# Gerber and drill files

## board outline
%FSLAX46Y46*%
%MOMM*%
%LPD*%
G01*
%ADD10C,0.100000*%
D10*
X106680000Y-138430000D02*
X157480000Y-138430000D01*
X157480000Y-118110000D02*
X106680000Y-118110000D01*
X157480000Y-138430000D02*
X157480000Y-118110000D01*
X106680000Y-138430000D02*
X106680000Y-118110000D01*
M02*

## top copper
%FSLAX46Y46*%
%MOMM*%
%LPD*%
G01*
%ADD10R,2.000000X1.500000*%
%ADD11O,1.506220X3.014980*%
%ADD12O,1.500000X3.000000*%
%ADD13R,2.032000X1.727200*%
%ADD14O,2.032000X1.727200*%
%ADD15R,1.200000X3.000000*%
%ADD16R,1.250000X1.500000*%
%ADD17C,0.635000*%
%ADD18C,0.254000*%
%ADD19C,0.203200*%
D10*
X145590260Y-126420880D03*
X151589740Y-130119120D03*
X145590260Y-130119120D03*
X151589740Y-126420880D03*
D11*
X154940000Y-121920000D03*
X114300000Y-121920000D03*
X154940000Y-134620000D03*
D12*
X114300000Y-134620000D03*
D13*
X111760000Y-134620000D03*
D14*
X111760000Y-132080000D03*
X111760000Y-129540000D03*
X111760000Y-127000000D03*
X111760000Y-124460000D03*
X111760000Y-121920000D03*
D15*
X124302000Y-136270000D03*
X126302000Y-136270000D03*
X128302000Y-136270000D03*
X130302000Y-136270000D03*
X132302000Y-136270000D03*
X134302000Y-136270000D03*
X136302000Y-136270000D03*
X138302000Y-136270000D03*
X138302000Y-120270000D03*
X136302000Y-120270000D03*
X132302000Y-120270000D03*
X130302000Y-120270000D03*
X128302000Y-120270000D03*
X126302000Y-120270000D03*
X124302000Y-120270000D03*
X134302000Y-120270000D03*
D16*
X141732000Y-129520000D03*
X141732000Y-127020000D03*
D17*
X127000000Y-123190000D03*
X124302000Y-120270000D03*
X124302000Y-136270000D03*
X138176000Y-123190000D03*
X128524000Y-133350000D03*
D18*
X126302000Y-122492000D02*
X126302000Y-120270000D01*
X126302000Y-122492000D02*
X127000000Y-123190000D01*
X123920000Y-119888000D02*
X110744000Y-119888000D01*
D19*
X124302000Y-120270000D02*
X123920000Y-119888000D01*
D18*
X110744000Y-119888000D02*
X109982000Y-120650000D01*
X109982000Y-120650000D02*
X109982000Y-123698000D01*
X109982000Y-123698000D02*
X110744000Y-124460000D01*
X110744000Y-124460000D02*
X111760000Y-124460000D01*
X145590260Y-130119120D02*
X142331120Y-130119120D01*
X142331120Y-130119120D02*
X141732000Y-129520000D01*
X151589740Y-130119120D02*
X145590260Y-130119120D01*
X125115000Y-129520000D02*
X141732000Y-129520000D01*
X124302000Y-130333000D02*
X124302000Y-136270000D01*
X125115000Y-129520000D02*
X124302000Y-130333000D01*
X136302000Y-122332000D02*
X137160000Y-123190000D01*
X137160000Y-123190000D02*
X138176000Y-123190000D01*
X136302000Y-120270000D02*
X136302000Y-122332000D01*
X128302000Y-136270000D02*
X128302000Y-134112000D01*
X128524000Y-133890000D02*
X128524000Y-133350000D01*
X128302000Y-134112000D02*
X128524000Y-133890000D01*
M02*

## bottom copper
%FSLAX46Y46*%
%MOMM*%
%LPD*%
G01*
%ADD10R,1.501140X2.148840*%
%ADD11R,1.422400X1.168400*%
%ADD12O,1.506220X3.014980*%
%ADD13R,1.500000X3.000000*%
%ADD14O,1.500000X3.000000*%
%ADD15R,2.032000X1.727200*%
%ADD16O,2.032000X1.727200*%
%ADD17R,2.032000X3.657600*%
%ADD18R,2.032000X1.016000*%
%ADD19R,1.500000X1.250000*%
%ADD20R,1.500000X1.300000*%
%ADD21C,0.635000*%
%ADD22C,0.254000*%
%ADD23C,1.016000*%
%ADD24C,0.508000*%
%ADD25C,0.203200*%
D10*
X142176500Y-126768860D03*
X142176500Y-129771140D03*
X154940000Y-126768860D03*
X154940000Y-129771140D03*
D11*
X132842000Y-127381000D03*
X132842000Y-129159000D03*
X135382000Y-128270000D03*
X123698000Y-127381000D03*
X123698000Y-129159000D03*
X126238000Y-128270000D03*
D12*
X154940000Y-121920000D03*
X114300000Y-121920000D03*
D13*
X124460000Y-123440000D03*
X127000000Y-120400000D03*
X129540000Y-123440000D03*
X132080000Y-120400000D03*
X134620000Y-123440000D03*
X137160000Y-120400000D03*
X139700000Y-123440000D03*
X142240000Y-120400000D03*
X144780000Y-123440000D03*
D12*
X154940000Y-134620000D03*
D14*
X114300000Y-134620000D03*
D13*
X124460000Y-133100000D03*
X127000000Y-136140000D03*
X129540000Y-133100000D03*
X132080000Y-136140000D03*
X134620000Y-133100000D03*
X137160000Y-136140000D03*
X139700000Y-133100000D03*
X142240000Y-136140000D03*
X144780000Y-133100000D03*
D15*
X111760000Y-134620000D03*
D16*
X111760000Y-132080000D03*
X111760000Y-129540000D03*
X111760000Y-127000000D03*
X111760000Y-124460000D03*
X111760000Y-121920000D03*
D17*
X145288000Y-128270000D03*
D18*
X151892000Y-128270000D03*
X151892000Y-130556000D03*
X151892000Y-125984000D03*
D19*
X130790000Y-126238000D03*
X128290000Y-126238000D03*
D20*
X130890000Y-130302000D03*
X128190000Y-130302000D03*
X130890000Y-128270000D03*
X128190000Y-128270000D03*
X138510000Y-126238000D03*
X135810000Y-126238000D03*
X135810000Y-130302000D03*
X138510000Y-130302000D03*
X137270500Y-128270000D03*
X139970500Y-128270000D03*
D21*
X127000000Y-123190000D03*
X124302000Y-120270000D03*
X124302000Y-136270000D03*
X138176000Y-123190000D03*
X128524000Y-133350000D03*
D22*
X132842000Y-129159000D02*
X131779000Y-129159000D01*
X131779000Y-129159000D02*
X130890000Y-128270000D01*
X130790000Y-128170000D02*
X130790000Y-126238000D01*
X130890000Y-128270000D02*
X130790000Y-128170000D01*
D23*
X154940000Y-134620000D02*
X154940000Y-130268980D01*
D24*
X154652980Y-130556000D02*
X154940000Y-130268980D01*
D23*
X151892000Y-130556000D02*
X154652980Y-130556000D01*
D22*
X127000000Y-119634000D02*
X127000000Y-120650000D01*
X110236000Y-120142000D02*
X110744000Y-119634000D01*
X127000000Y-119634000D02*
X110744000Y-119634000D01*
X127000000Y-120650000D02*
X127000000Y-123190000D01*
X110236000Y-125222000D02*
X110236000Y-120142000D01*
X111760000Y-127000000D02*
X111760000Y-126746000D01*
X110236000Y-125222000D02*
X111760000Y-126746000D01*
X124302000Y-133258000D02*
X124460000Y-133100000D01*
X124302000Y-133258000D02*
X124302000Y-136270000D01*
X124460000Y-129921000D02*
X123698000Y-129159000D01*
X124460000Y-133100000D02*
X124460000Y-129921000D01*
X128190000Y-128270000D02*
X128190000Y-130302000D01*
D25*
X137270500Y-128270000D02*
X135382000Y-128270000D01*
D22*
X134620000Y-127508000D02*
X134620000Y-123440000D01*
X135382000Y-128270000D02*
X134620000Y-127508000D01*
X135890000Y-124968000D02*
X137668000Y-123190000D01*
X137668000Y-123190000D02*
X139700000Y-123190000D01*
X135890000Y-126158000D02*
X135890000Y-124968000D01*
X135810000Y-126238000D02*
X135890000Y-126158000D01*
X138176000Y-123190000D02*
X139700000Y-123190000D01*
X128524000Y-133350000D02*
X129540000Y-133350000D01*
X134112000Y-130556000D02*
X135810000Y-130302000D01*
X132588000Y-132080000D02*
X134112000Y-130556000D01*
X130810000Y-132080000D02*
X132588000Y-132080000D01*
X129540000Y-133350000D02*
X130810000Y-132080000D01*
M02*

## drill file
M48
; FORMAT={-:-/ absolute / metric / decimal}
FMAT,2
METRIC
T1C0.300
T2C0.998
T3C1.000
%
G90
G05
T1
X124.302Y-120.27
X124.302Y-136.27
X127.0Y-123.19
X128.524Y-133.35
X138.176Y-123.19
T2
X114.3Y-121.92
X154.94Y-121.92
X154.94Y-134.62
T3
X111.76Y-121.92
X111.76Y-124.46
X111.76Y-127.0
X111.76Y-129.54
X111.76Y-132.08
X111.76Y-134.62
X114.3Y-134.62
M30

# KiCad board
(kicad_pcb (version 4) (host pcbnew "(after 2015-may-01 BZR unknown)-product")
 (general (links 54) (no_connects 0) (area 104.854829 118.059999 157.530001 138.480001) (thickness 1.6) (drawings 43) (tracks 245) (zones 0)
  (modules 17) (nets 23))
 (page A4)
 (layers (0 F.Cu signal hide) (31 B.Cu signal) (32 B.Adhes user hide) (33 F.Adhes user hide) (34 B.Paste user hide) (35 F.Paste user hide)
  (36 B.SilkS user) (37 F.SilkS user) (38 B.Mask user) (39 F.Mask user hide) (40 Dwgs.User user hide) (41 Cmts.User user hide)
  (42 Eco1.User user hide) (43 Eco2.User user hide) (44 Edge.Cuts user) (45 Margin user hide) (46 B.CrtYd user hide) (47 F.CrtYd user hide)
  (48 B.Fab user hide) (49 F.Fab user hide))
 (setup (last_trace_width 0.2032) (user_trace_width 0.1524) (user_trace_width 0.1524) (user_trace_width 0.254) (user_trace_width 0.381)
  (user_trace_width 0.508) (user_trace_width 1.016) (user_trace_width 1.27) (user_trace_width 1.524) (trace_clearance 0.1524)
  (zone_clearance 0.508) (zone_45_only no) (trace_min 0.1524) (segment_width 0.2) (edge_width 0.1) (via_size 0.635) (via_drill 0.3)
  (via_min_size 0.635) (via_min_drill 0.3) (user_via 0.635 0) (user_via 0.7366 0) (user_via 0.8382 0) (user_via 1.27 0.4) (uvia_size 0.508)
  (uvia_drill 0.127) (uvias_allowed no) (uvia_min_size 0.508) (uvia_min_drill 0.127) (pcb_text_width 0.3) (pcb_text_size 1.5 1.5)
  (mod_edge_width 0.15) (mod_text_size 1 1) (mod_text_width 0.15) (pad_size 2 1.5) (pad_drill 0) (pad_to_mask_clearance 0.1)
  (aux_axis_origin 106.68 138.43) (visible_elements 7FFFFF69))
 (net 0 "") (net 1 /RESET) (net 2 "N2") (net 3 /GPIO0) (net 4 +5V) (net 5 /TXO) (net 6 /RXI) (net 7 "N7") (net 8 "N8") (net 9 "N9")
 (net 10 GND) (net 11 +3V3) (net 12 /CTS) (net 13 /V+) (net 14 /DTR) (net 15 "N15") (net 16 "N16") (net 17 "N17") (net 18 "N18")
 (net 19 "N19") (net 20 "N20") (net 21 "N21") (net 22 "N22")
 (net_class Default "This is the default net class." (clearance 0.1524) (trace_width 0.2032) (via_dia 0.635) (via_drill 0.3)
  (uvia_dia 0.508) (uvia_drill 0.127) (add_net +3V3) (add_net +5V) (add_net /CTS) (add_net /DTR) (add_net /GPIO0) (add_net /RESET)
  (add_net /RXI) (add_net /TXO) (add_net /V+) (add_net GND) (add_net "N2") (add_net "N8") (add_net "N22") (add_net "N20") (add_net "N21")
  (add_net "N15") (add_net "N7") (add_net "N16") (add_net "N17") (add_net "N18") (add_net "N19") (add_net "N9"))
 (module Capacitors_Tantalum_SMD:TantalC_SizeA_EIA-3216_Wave (layer B.Cu) (at 142.1765 128.27 90)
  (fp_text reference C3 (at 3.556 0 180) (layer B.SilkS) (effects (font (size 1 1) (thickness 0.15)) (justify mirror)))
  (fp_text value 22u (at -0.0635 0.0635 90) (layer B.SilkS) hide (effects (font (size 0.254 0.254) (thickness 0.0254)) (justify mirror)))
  (pad 2 smd rect (at 1.50114 0 90) (size 2.14884 1.50114) (layers B.Cu B.Paste B.Mask))
  (pad 1 smd rect (at -1.50114 0 90) (size 2.14884 1.50114) (layers B.Cu B.Paste B.Mask)))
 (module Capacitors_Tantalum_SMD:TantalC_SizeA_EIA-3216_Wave (layer B.Cu) (at 154.94 128.27 90)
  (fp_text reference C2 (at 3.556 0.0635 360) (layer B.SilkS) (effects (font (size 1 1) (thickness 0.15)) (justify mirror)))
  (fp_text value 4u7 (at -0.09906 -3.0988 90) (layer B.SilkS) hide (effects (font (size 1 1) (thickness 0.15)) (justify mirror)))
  (pad 2 smd rect (at 1.50114 0 90) (size 2.14884 1.50114) (layers B.Cu B.Paste B.Mask))
  (pad 1 smd rect (at -1.50114 0 90) (size 2.14884 1.50114) (layers B.Cu B.Paste B.Mask)))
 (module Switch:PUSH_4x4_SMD (layer F.Cu) (at 148.59 128.27) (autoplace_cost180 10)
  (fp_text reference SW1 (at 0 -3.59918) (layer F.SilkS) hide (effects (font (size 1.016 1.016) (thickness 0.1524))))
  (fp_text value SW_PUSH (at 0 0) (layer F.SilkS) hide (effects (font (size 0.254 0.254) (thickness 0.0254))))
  (pad 1 smd rect (at -2.99974 -1.84912) (size 2 1.5) (layers F.Cu F.Paste F.Mask))
  (pad 2 smd rect (at 2.99974 1.84912) (size 2 1.5) (layers F.Cu F.Paste F.Mask) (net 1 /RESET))
  (pad 2 smd rect (at -2.99974 1.84912) (size 2 1.5) (layers F.Cu F.Paste F.Mask) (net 1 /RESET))
  (pad 1 smd rect (at 2.99974 -1.84912) (size 2 1.5) (layers F.Cu F.Paste F.Mask)))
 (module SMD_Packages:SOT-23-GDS (layer B.Cu) (at 134.112 128.27 270)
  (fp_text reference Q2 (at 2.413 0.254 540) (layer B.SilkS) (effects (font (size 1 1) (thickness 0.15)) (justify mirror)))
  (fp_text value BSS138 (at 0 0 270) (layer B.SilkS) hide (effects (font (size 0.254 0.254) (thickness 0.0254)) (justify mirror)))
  (pad S smd rect (at -0.889 1.27 270) (size 1.1684 1.4224) (layers B.Cu B.Paste B.Mask))
  (pad G smd rect (at 0.889 1.27 270) (size 1.1684 1.4224) (layers B.Cu B.Paste B.Mask) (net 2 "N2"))
  (pad D smd rect (at 0 -1.27 270) (size 1.1684 1.4224) (layers B.Cu B.Paste B.Mask) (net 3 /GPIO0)))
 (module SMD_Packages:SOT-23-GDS (layer B.Cu) (at 124.968 128.27 270)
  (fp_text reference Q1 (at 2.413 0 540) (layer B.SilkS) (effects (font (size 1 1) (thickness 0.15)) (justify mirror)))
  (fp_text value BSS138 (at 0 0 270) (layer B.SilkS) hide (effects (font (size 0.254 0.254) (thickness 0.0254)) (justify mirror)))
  (pad S smd rect (at -0.889 1.27 270) (size 1.1684 1.4224) (layers B.Cu B.Paste B.Mask))
  (pad G smd rect (at 0.889 1.27 270) (size 1.1684 1.4224) (layers B.Cu B.Paste B.Mask) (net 1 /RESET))
  (pad D smd rect (at 0 -1.27 270) (size 1.1684 1.4224) (layers B.Cu B.Paste B.Mask)))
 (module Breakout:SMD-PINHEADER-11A (layer B.Cu) (at 114.3 121.92)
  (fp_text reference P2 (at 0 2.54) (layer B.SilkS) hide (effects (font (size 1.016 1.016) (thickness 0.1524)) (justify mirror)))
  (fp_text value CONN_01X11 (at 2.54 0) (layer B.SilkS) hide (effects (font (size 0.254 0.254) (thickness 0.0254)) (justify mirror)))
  (pad 11 thru_hole oval (at 40.64 0) (size 1.50622 3.01498) (drill 0.99822) (layers *.Cu *.Mask))
  (pad 1 thru_hole oval (at 0 0) (size 1.50622 3.01498) (drill 0.99822) (layers *.Cu *.Mask))
  (pad 2 smd rect (at 10.16 1.52) (size 1.5 3) (layers B.Cu B.Paste B.Mask))
  (pad 3 smd rect (at 12.7 -1.52) (size 1.5 3) (layers B.Cu B.Paste B.Mask))
  (pad 4 smd rect (at 15.24 1.52) (size 1.5 3) (layers B.Cu B.Paste B.Mask))
  (pad 5 smd rect (at 17.78 -1.52) (size 1.5 3) (layers B.Cu B.Paste B.Mask))
  (pad 6 smd rect (at 20.32 1.52) (size 1.5 3) (layers B.Cu B.Paste B.Mask) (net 3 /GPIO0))
  (pad 7 smd rect (at 22.86 -1.52) (size 1.5 3) (layers B.Cu B.Paste B.Mask))
  (pad 8 smd rect (at 25.4 1.52) (size 1.5 3) (layers B.Cu B.Paste B.Mask))
  (pad 9 smd rect (at 27.94 -1.52) (size 1.5 3) (layers B.Cu B.Paste B.Mask))
  (pad 10 smd rect (at 30.48 1.52) (size 1.5 3) (layers B.Cu B.Paste B.Mask)))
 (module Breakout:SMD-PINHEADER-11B (layer B.Cu) (at 114.3 134.62)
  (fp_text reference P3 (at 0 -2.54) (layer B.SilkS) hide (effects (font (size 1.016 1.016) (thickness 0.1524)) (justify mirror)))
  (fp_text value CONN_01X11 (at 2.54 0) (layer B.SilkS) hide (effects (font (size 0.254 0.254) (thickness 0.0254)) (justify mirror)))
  (pad 11 thru_hole oval (at 40.64 0) (size 1.50622 3.01498) (drill 0.99822) (layers *.Cu *.Mask) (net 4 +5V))
  (pad 1 thru_hole oval (at 0 0) (size 1.5 3) (drill 1) (layers *.Cu *.Mask))
  (pad 2 smd rect (at 10.16 -1.52) (size 1.5 3) (layers B.Cu B.Paste B.Mask) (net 1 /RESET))
  (pad 3 smd rect (at 12.7 1.52) (size 1.5 3) (layers B.Cu B.Paste B.Mask))
  (pad 4 smd rect (at 15.24 -1.52) (size 1.5 3) (layers B.Cu B.Paste B.Mask))
  (pad 5 smd rect (at 17.78 1.52) (size 1.5 3) (layers B.Cu B.Paste B.Mask))
  (pad 6 smd rect (at 20.32 -1.52) (size 1.5 3) (layers B.Cu B.Paste B.Mask))
  (pad 7 smd rect (at 22.86 1.52) (size 1.5 3) (layers B.Cu B.Paste B.Mask))
  (pad 8 smd rect (at 25.4 -1.52) (size 1.5 3) (layers B.Cu B.Paste B.Mask))
  (pad 9 smd rect (at 27.94 1.52) (size 1.5 3) (layers B.Cu B.Paste B.Mask))
  (pad 10 smd rect (at 30.48 -1.52) (size 1.5 3) (layers B.Cu B.Paste B.Mask)))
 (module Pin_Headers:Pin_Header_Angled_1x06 (layer F.Cu) (at 111.76 128.27 90)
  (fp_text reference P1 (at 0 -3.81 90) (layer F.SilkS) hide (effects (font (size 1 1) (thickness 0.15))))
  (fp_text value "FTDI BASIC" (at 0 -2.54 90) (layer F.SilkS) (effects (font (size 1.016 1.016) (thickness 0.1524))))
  (pad 1 thru_hole rect (at -6.35 0 90) (size 1.7272 2.032) (drill 1) (layers *.Cu *.Mask F.SilkS))
  (pad 2 thru_hole oval (at -3.81 0 90) (size 1.7272 2.032) (drill 1) (layers *.Cu *.Mask F.SilkS))
  (pad 3 thru_hole oval (at -1.27 0 90) (size 1.7272 2.032) (drill 1) (layers *.Cu *.Mask F.SilkS))
  (pad 4 thru_hole oval (at 1.27 0 90) (size 1.7272 2.032) (drill 1) (layers *.Cu *.Mask F.SilkS) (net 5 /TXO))
  (pad 5 thru_hole oval (at 3.81 0 90) (size 1.7272 2.032) (drill 1) (layers *.Cu *.Mask F.SilkS) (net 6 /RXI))
  (pad 6 thru_hole oval (at 6.35 0 90) (size 1.7272 2.032) (drill 1) (layers *.Cu *.Mask F.SilkS)))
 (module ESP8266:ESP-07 (layer F.Cu) (at 130.302 128.27)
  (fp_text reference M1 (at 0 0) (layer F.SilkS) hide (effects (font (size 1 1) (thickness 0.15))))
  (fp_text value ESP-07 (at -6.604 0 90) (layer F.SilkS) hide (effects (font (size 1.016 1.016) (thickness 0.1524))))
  (pad 1 smd rect (at -6 8) (size 1.2 3) (layers F.Cu F.Paste F.Mask) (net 1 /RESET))
  (pad 2 smd rect (at -4 8) (size 1.2 3) (layers F.Cu F.Paste F.Mask))
  (pad 3 smd rect (at -2 8) (size 1.2 3) (layers F.Cu F.Paste F.Mask) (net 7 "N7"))
  (pad 4 smd rect (at 0 8) (size 1.2 3) (layers F.Cu F.Paste F.Mask))
  (pad 5 smd rect (at 2 8) (size 1.2 3) (layers F.Cu F.Paste F.Mask))
  (pad 6 smd rect (at 4 8) (size 1.2 3) (layers F.Cu F.Paste F.Mask))
  (pad 7 smd rect (at 6 8) (size 1.2 3) (layers F.Cu F.Paste F.Mask))
  (pad 8 smd rect (at 8 8) (size 1.2 3) (layers F.Cu F.Paste F.Mask))
  (pad 9 smd rect (at 8 -8) (size 1.2 3) (layers F.Cu F.Paste F.Mask))
  (pad 10 smd rect (at 6 -8) (size 1.2 3) (layers F.Cu F.Paste F.Mask) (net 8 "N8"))
  (pad 12 smd rect (at 2 -8) (size 1.2 3) (layers F.Cu F.Paste F.Mask))
  (pad 13 smd rect (at 0 -8) (size 1.2 3) (layers F.Cu F.Paste F.Mask))
  (pad 14 smd rect (at -2 -8) (size 1.2 3) (layers F.Cu F.Paste F.Mask))
  (pad 15 smd rect (at -4 -8) (size 1.2 3) (layers F.Cu F.Paste F.Mask) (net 5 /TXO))
  (pad 16 smd rect (at -6 -8) (size 1.2 3) (layers F.Cu F.Paste F.Mask) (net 6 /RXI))
  (pad 11 smd rect (at 4 -8) (size 1.2 3) (layers F.Cu F.Paste F.Mask)))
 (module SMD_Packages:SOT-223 (layer B.Cu) (at 148.59 128.27 270)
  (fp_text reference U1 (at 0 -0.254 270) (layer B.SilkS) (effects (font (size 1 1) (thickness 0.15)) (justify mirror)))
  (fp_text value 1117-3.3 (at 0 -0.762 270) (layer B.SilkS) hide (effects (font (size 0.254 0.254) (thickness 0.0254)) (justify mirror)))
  (pad 2 smd rect (at 0 3.302 270) (size 3.6576 2.032) (layers B.Cu B.Paste B.Mask))
  (pad 2 smd rect (at 0 -3.302 270) (size 1.016 2.032) (layers B.Cu B.Paste B.Mask))
  (pad 3 smd rect (at 2.286 -3.302 270) (size 1.016 2.032) (layers B.Cu B.Paste B.Mask) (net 4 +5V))
  (pad 1 smd rect (at -2.286 -3.302 270) (size 1.016 2.032) (layers B.Cu B.Paste B.Mask)))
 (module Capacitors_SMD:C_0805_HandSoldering (layer B.Cu) (at 129.54 126.238 180)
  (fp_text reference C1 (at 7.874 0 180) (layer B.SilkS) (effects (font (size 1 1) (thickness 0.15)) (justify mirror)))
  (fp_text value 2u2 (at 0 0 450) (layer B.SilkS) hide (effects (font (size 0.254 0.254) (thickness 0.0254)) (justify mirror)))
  (pad 1 smd rect (at -1.25 0 180) (size 1.5 1.25) (layers B.Cu B.Paste B.Mask) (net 2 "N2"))
  (pad 2 smd rect (at 1.25 0 180) (size 1.5 1.25) (layers B.Cu B.Paste B.Mask)))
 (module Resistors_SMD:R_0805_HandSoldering (layer B.Cu) (at 129.54 130.302 180)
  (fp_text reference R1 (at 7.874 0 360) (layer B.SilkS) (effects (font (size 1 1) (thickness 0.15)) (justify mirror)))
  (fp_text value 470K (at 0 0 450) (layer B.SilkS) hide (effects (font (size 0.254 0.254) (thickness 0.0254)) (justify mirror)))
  (pad 1 smd rect (at -1.35 0 180) (size 1.5 1.3) (layers B.Cu B.Paste B.Mask))
  (pad 2 smd rect (at 1.35 0 180) (size 1.5 1.3) (layers B.Cu B.Paste B.Mask) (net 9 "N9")))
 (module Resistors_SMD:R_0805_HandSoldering (layer B.Cu) (at 129.54 128.27 180)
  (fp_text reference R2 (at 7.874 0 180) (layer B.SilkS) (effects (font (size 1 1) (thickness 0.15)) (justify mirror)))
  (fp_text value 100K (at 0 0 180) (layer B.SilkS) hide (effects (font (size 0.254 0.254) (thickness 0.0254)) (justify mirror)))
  (pad 1 smd rect (at -1.35 0 180) (size 1.5 1.3) (layers B.Cu B.Paste B.Mask) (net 2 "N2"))
  (pad 2 smd rect (at 1.35 0 180) (size 1.5 1.3) (layers B.Cu B.Paste B.Mask) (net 9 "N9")))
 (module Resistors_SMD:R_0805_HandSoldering (layer B.Cu) (at 137.16 126.238 180)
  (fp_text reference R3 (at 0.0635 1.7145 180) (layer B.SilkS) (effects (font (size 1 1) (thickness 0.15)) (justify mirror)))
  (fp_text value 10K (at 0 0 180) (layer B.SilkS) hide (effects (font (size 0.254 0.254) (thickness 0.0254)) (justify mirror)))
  (pad 1 smd rect (at -1.35 0 180) (size 1.5 1.3) (layers B.Cu B.Paste B.Mask))
  (pad 2 smd rect (at 1.35 0 180) (size 1.5 1.3) (layers B.Cu B.Paste B.Mask) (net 8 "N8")))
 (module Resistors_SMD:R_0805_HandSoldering (layer B.Cu) (at 137.16 130.302)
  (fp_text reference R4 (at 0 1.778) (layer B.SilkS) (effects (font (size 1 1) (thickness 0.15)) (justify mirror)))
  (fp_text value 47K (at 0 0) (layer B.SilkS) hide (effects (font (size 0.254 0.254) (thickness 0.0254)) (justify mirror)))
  (pad 1 smd rect (at -1.35 0) (size 1.5 1.3) (layers B.Cu B.Paste B.Mask) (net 7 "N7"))
  (pad 2 smd rect (at 1.35 0) (size 1.5 1.3) (layers B.Cu B.Paste B.Mask)))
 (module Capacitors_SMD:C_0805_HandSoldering (layer F.Cu) (at 141.732 128.27 90)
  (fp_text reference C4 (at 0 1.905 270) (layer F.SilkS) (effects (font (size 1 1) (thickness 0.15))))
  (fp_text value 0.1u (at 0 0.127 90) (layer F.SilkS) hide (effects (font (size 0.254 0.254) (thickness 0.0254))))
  (pad 1 smd rect (at -1.25 0 90) (size 1.5 1.25) (layers F.Cu F.Paste F.Mask) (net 1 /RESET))
  (pad 2 smd rect (at 1.25 0 90) (size 1.5 1.25) (layers F.Cu F.Paste F.Mask)))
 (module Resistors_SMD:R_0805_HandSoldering (layer B.Cu) (at 138.6205 128.27)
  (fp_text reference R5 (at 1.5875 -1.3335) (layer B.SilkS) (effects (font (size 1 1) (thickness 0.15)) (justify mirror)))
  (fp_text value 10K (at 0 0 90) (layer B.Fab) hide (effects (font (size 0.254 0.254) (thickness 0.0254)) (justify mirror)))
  (pad 1 smd rect (at -1.35 0) (size 1.5 1.3) (layers B.Cu B.Paste B.Mask) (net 3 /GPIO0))
  (pad 2 smd rect (at 1.35 0) (size 1.5 1.3) (layers B.Cu B.Paste B.Mask)))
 (gr_line (start 106.68 138.43) (end 157.48 138.43) (angle 90) (layer Edge.Cuts) (width 0.1))
 (gr_line (start 157.48 118.11) (end 106.68 118.11) (angle 90) (layer Edge.Cuts) (width 0.1))
 (gr_line (start 157.48 138.43) (end 157.48 118.11) (angle 90) (layer Edge.Cuts) (width 0.1))
 (gr_line (start 106.68 138.43) (end 106.68 118.11) (angle 90) (layer Edge.Cuts) (width 0.1))
 (segment (start 132.842 129.159) (end 131.779 129.159) (width 0.254) (layer B.Cu) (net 2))
 (segment (start 131.779 129.159) (end 130.89 128.27) (width 0.254) (layer B.Cu) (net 2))
 (segment (start 130.79 128.17) (end 130.79 126.238) (width 0.254) (layer B.Cu) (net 2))
 (segment (start 130.89 128.27) (end 130.79 128.17) (width 0.254) (layer B.Cu) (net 2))
 (segment (start 154.94 134.62) (end 154.94 130.26898) (width 1.016) (layer B.Cu) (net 4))
 (segment (start 154.65298 130.556) (end 154.94 130.26898) (width 0.508) (layer B.Cu) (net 4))
 (segment (start 151.892 130.556) (end 154.65298 130.556) (width 1.016) (layer B.Cu) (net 4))
 (segment (start 127 119.634) (end 127 120.65) (width 0.254) (layer B.Cu) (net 5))
 (segment (start 110.236 120.142) (end 110.744 119.634) (width 0.254) (layer B.Cu) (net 5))
 (segment (start 127 119.634) (end 110.744 119.634) (width 0.254) (layer B.Cu) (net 5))
 (segment (start 126.302 122.492) (end 126.302 120.27) (width 0.254) (layer F.Cu) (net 5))
 (segment (start 126.302 122.492) (end 127 123.19) (width 0.254) (layer F.Cu) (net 5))
 (segment (start 127 120.65) (end 127 123.19) (width 0.254) (layer B.Cu) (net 5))
 (segment (start 110.236 125.222) (end 110.236 120.142) (width 0.254) (layer B.Cu) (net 5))
 (segment (start 111.76 127) (end 111.76 126.746) (width 0.254) (layer B.Cu) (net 5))
 (segment (start 110.236 125.222) (end 111.76 126.746) (width 0.254) (layer B.Cu) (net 5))
 (segment (start 123.92 119.888) (end 110.744 119.888) (width 0.254) (layer F.Cu) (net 6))
 (segment (start 124.302 120.27) (end 123.92 119.888) (width 0.2032) (layer F.Cu) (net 6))
 (segment (start 110.744 119.888) (end 109.982 120.65) (width 0.254) (layer F.Cu) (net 6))
 (segment (start 109.982 120.65) (end 109.982 123.698) (width 0.254) (layer F.Cu) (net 6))
 (segment (start 109.982 123.698) (end 110.744 124.46) (width 0.254) (layer F.Cu) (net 6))
 (segment (start 110.744 124.46) (end 111.76 124.46) (width 0.254) (layer F.Cu) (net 6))
 (segment (start 145.59026 130.11912) (end 142.33112 130.11912) (width 0.254) (layer F.Cu) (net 1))
 (segment (start 142.33112 130.11912) (end 141.732 129.52) (width 0.254) (layer F.Cu) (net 1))
 (segment (start 151.58974 130.11912) (end 145.59026 130.11912) (width 0.254) (layer F.Cu) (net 1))
 (segment (start 124.302 133.258) (end 124.46 133.1) (width 0.254) (layer B.Cu) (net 1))
 (segment (start 125.115 129.52) (end 141.732 129.52) (width 0.254) (layer F.Cu) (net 1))
 (segment (start 124.302 130.333) (end 124.302 136.27) (width 0.254) (layer F.Cu) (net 1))
 (segment (start 125.115 129.52) (end 124.302 130.333) (width 0.254) (layer F.Cu) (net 1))
 (segment (start 124.302 133.258) (end 124.302 136.27) (width 0.254) (layer B.Cu) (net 1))
 (segment (start 124.46 129.921) (end 123.698 129.159) (width 0.254) (layer B.Cu) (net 1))
 (segment (start 124.46 133.1) (end 124.46 129.921) (width 0.254) (layer B.Cu) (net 1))
 (segment (start 128.19 128.27) (end 128.19 130.302) (width 0.254) (layer B.Cu) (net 9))
 (segment (start 137.2705 128.27) (end 135.382 128.27) (width 0.2032) (layer B.Cu) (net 3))
 (segment (start 134.62 127.508) (end 134.62 123.44) (width 0.254) (layer B.Cu) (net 3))
 (segment (start 135.382 128.27) (end 134.62 127.508) (width 0.254) (layer B.Cu) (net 3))
 (segment (start 135.89 124.968) (end 137.668 123.19) (width 0.254) (layer B.Cu) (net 8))
 (segment (start 137.668 123.19) (end 139.7 123.19) (width 0.254) (layer B.Cu) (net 8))
 (segment (start 135.89 126.158) (end 135.89 124.968) (width 0.254) (layer B.Cu) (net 8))
 (segment (start 135.81 126.238) (end 135.89 126.158) (width 0.254) (layer B.Cu) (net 8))
 (segment (start 136.302 122.332) (end 137.16 123.19) (width 0.254) (layer F.Cu) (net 8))
 (segment (start 137.16 123.19) (end 138.176 123.19) (width 0.254) (layer F.Cu) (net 8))
 (segment (start 138.176 123.19) (end 139.7 123.19) (width 0.254) (layer B.Cu) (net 8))
 (segment (start 136.302 120.27) (end 136.302 122.332) (width 0.254) (layer F.Cu) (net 8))
 (segment (start 128.524 133.35) (end 129.54 133.35) (width 0.254) (layer B.Cu) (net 7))
 (segment (start 128.302 136.27) (end 128.302 134.112) (width 0.254) (layer F.Cu) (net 7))
 (segment (start 134.112 130.556) (end 135.81 130.302) (width 0.254) (layer B.Cu) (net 7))
 (segment (start 132.588 132.08) (end 134.112 130.556) (width 0.254) (layer B.Cu) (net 7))
 (segment (start 130.81 132.08) (end 132.588 132.08) (width 0.254) (layer B.Cu) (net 7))
 (segment (start 129.54 133.35) (end 130.81 132.08) (width 0.254) (layer B.Cu) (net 7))
 (segment (start 128.524 133.89) (end 128.524 133.35) (width 0.254) (layer F.Cu) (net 7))
 (segment (start 128.302 134.112) (end 128.524 133.89) (width 0.254) (layer F.Cu) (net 7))
 (via (at 127 123.19) (size 0.635) (layers F.Cu B.Cu) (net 5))
 (via (at 124.302 120.27) (size 0.635) (layers F.Cu B.Cu) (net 6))
 (via (at 124.302 136.27) (size 0.635) (layers F.Cu B.Cu) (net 1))
 (via (at 138.176 123.19) (size 0.635) (layers F.Cu B.Cu) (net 8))
 (via (at 128.524 133.35) (size 0.635) (layers F.Cu B.Cu) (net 7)))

